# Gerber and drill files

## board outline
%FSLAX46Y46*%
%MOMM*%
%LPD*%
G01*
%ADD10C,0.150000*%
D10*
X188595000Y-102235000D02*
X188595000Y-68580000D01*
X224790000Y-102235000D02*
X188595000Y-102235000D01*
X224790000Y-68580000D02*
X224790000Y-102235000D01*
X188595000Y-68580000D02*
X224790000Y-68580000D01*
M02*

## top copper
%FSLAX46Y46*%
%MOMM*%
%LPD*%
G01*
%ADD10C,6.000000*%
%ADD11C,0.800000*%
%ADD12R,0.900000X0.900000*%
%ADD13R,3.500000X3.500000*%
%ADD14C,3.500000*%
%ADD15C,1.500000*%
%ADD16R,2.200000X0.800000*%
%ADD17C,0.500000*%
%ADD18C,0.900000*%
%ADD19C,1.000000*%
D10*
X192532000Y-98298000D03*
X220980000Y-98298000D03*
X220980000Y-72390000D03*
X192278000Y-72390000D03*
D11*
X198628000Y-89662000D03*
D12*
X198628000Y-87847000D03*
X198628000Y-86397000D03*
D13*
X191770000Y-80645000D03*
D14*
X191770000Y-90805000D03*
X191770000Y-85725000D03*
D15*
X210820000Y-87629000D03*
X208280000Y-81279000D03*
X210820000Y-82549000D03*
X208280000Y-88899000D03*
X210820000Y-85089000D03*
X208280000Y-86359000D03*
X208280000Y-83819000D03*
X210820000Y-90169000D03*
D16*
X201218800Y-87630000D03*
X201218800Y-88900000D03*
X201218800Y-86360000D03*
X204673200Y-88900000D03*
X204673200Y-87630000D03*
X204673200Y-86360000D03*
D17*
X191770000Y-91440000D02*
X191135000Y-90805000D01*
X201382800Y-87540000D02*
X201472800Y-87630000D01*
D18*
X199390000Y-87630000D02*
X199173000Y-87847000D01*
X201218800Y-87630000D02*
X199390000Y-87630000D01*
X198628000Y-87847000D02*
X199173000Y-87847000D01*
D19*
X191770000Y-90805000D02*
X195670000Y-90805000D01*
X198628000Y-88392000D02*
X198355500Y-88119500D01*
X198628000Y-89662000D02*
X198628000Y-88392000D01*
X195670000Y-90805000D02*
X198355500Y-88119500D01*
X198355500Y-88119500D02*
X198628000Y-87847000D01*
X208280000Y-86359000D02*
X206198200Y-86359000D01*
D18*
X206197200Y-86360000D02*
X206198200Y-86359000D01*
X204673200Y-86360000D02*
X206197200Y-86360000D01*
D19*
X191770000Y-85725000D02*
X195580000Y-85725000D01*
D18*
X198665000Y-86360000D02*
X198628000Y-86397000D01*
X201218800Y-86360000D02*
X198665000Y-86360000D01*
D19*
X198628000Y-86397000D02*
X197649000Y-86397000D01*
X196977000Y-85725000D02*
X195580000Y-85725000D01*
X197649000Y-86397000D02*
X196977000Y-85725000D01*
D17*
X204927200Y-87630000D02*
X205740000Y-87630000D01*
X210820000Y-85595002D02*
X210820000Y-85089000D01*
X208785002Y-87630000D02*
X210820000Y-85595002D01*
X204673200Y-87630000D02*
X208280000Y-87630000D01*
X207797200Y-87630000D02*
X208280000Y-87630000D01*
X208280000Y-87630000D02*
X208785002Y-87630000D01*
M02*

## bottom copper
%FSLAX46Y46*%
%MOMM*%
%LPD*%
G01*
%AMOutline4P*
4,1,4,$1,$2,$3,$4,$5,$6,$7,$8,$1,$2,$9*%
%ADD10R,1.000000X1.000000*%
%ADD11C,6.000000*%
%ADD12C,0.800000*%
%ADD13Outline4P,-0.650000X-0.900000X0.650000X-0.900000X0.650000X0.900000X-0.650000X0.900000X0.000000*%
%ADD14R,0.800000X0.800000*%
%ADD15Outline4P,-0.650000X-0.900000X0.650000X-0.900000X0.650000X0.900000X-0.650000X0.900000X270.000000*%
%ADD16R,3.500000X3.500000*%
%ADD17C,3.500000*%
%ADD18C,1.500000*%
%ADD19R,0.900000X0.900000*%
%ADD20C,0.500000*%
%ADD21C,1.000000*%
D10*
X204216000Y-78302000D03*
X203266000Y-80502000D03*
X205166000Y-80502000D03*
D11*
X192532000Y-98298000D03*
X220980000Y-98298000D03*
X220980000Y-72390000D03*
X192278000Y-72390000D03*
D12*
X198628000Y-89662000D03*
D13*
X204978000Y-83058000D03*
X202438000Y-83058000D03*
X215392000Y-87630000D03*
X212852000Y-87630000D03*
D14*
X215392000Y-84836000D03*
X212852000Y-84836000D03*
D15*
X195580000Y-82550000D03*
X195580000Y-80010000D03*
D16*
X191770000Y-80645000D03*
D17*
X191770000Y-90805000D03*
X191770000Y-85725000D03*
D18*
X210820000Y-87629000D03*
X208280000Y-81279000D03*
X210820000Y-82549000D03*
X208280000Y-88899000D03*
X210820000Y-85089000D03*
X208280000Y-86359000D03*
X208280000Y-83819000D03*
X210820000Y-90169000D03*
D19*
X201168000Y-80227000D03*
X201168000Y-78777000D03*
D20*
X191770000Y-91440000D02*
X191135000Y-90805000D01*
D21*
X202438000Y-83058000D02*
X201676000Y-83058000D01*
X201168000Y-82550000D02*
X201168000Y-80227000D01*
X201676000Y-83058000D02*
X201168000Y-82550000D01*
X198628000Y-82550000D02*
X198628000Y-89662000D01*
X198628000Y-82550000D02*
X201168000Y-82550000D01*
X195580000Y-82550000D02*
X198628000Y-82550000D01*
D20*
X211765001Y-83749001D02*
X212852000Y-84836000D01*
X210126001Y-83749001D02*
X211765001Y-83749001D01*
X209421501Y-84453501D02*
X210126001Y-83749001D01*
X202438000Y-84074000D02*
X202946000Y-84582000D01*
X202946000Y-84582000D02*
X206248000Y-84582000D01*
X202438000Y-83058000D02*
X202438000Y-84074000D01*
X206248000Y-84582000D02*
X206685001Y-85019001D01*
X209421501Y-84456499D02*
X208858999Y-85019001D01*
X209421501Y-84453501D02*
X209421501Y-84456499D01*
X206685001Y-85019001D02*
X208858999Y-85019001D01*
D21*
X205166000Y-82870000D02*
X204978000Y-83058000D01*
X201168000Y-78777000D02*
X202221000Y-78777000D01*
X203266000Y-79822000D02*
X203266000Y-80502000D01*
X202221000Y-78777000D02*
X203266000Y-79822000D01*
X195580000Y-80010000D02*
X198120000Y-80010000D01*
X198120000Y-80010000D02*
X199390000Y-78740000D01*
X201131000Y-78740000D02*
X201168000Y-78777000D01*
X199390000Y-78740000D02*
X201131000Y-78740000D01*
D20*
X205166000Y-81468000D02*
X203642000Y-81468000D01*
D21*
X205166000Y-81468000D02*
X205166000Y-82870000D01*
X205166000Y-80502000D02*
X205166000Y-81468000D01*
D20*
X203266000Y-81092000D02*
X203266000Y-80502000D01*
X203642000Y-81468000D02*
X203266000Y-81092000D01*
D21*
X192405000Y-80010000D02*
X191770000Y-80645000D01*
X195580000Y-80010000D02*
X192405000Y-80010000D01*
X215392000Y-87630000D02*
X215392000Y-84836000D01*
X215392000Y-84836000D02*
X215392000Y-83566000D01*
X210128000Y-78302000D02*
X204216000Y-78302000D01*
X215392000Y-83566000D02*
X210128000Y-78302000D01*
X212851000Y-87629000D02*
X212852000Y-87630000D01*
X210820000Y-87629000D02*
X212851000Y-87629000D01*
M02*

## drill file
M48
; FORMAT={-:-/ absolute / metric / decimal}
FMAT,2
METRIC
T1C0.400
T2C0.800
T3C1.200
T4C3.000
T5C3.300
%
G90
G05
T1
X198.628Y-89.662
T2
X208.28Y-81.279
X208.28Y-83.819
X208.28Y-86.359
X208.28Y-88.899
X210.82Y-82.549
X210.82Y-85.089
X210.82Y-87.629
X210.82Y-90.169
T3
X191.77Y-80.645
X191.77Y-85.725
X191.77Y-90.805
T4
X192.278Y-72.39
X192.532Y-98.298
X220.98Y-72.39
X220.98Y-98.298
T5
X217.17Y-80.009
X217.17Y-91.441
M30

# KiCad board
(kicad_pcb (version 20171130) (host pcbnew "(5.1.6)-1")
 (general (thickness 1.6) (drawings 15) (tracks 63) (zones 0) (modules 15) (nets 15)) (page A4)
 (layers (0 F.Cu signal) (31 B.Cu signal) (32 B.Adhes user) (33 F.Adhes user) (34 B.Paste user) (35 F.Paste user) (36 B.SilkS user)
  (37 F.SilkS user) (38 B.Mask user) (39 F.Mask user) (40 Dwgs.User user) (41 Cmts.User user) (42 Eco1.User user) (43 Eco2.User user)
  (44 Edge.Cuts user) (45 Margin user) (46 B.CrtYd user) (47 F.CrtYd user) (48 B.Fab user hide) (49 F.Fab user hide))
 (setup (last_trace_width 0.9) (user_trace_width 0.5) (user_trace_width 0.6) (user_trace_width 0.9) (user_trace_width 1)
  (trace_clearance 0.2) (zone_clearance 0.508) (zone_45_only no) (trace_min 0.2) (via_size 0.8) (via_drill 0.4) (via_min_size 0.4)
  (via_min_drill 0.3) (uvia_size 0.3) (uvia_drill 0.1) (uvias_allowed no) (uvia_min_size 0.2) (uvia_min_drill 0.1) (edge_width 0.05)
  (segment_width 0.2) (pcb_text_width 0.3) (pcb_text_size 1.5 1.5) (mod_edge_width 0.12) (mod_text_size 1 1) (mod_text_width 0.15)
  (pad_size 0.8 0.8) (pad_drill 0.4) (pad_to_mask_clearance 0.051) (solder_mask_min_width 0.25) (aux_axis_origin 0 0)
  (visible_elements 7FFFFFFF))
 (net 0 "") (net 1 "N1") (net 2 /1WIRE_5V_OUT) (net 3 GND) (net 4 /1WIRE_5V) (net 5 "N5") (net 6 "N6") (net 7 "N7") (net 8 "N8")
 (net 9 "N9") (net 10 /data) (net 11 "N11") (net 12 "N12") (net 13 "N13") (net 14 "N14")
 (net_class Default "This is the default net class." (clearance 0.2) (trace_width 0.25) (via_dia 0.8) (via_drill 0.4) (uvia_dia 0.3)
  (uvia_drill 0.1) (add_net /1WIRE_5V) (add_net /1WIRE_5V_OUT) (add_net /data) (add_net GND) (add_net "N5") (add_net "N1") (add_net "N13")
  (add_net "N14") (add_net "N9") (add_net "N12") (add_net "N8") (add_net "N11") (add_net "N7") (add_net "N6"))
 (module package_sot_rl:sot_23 (layer B.Cu) (at 204.216 79.502 90)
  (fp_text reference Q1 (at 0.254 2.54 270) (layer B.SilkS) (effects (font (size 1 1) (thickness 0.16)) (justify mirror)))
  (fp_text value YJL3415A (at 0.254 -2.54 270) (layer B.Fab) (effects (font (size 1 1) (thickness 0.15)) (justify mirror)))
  (pad 3 smd rect (at 1.2 0 90) (size 1 1) (layers B.Cu B.Paste B.Mask) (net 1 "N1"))
  (pad 2 smd rect (at -1 -0.95 90) (size 1 1) (layers B.Cu B.Paste B.Mask) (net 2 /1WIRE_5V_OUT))
  (pad 1 smd rect (at -1 0.95 90) (size 1 1) (layers B.Cu B.Paste B.Mask) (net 2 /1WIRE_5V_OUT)))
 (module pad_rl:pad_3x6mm (layer F.Cu) (at 192.532 98.298)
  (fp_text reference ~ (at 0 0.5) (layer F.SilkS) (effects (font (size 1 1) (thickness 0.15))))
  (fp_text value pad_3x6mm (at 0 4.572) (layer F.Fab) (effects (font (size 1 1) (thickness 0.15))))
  (pad ~ thru_hole circle (at 0 0) (size 6 6) (drill 3) (layers *.Cu *.Mask)))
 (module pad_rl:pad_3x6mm (layer F.Cu) (at 220.98 98.298)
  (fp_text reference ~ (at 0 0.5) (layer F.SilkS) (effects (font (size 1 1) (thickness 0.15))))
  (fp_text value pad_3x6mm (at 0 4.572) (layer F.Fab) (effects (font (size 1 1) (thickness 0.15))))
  (pad ~ thru_hole circle (at 0 0) (size 6 6) (drill 3) (layers *.Cu *.Mask)))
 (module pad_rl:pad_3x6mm (layer F.Cu) (at 220.98 72.39)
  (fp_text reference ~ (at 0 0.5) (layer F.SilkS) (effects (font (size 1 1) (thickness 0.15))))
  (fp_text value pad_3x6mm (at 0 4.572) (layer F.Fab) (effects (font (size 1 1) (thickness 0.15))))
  (pad ~ thru_hole circle (at 0 0) (size 6 6) (drill 3) (layers *.Cu *.Mask)))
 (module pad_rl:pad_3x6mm (layer F.Cu) (at 192.278 72.39)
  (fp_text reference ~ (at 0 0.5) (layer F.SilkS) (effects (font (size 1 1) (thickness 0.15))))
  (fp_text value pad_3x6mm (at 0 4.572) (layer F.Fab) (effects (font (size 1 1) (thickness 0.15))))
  (pad ~ thru_hole circle (at 0 0) (size 6 6) (drill 3) (layers *.Cu *.Mask)))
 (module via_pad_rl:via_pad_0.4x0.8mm (layer F.Cu) (at 198.628 89.662)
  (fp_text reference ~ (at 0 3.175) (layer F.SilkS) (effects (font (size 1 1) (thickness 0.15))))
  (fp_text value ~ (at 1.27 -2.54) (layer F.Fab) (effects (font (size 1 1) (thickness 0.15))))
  (pad ~ thru_hole circle (at 0 0) (size 0.8 0.8) (drill 0.4) (layers *.Cu *.Mask) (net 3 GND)))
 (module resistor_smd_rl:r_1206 (layer B.Cu) (at 203.708 83.058)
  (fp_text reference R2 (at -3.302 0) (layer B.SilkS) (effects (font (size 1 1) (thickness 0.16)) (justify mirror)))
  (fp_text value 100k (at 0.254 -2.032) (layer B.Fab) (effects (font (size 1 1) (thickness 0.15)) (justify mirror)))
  (pad 2 smd trapezoid (at 1.27 0) (size 1.3 1.8) (layers B.Cu B.Paste B.Mask) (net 2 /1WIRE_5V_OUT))
  (pad 1 smd trapezoid (at -1.27 0) (size 1.3 1.8) (layers B.Cu B.Paste B.Mask) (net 3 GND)))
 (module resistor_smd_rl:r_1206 (layer B.Cu) (at 214.122 87.63)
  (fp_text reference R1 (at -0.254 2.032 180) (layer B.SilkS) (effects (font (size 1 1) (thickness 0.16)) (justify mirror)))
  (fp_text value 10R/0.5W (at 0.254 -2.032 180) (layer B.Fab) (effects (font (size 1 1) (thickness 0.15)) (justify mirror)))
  (pad 2 smd trapezoid (at 1.27 0) (size 1.3 1.8) (layers B.Cu B.Paste B.Mask) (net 1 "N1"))
  (pad 1 smd trapezoid (at -1.27 0) (size 1.3 1.8) (layers B.Cu B.Paste B.Mask) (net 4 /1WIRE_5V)))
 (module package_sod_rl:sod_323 (layer B.Cu) (at 214.122 84.836 180)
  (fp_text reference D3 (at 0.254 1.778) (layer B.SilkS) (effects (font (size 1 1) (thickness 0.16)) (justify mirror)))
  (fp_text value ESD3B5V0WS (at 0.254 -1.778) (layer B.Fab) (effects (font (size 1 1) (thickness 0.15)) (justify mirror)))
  (pad 1 smd rect (at -1.27 0 180) (size 0.8 0.8) (layers B.Cu B.Paste B.Mask) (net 1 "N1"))
  (pad 2 smd rect (at 1.27 0 180) (size 0.8 0.8) (layers B.Cu B.Paste B.Mask) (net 3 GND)))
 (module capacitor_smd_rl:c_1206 (layer B.Cu) (at 195.58 81.28 270)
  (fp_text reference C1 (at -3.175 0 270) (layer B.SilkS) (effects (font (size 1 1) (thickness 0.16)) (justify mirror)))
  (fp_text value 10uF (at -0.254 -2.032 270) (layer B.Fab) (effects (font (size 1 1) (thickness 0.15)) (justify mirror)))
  (pad 2 smd trapezoid (at 1.27 0 270) (size 1.3 1.8) (layers B.Cu B.Paste B.Mask) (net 3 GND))
  (pad 1 smd trapezoid (at -1.27 0 270) (size 1.3 1.8) (layers B.Cu B.Paste B.Mask) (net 2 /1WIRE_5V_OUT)))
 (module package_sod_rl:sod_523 (layer F.Cu) (at 198.628 87.122 270)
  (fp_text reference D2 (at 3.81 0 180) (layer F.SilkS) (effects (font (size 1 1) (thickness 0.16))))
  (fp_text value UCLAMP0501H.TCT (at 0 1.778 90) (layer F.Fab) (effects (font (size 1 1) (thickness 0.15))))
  (pad 2 smd rect (at 0.725 0 270) (size 0.9 0.9) (layers F.Cu F.Paste F.Mask) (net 3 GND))
  (pad 1 smd rect (at -0.725 0 270) (size 0.9 0.9) (layers F.Cu F.Paste F.Mask) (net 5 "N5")))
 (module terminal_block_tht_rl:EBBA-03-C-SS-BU (layer F.Cu) (at 191.77 85.725 270)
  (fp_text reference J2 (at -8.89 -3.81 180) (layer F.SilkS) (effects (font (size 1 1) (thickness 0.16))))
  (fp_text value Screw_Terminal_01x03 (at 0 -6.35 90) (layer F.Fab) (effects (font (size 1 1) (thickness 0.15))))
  (pad 1 thru_hole rect (at -5.08 0 90) (size 3.5 3.5) (drill 1.2) (layers *.Cu *.Mask) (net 2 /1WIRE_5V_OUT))
  (pad 3 thru_hole circle (at 5.08 0 90) (size 3.5 3.5) (drill 1.2) (layers *.Cu *.Mask) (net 3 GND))
  (pad 2 thru_hole circle (at 0 0 90) (size 3.5 3.5) (drill 1.2) (layers *.Cu *.Mask) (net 5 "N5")))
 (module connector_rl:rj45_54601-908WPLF (layer F.Cu) (at 217.17 85.725 90)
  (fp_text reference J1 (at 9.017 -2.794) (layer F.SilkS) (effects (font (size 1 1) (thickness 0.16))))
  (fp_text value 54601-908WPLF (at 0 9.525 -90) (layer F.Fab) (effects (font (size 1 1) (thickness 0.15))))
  (pad 3 thru_hole circle (at -1.904 -6.35 90) (size 1.5 1.5) (drill 0.8) (layers *.Cu *.Mask) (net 4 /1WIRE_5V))
  (pad 8 thru_hole circle (at 4.446 -8.89 90) (size 1.5 1.5) (drill 0.8) (layers *.Cu *.Mask) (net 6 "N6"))
  (pad "" np_thru_hole circle (at -5.716 0 90) (size 3.3 3.3) (drill 3.3) (layers *.Cu *.SilkS *.Mask))
  (pad 7 thru_hole circle (at 3.176 -6.35 90) (size 1.5 1.5) (drill 0.8) (layers *.Cu *.Mask) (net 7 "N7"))
  (pad 2 thru_hole circle (at -3.174 -8.89 90) (size 1.5 1.5) (drill 0.8) (layers *.Cu *.Mask) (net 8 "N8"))
  (pad 5 thru_hole circle (at 0.636 -6.35 90) (size 1.5 1.5) (drill 0.8) (layers *.Cu *.Mask) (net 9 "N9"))
  (pad 4 thru_hole circle (at -0.634 -8.89 90) (size 1.5 1.5) (drill 0.8) (layers *.Cu *.Mask) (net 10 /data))
  (pad 6 thru_hole circle (at 1.906 -8.89 270) (size 1.5 1.5) (drill 0.8) (layers *.Cu *.Mask) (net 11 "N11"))
  (pad 1 thru_hole circle (at -4.444 -6.35 90) (size 1.5 1.5) (drill 0.8) (layers *.Cu *.Mask) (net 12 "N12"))
  (pad "" np_thru_hole circle (at 5.716 0 90) (size 3.3 3.3) (drill 3.3) (layers *.Cu *.SilkS *.Mask)))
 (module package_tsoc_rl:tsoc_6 (layer F.Cu) (at 202.946 87.63)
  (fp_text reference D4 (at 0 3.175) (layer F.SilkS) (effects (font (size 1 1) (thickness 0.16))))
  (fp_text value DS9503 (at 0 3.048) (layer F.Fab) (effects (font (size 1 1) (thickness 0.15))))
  (pad 2 smd rect (at -1.7272 0) (size 2.2 0.8) (layers F.Cu F.Paste F.Mask) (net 3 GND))
  (pad 3 smd rect (at -1.7272 1.27) (size 2.2 0.8) (layers F.Cu F.Paste F.Mask) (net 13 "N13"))
  (pad 1 smd rect (at -1.7272 -1.27) (size 2.2 0.8) (layers F.Cu F.Paste F.Mask) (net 5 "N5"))
  (pad 4 smd rect (at 1.7272 1.27) (size 2.2 0.8) (layers F.Cu F.Paste F.Mask) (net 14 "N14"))
  (pad 5 smd rect (at 1.7272 0) (size 2.2 0.8) (layers F.Cu F.Paste F.Mask) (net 9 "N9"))
  (pad 6 smd rect (at 1.7272 -1.27) (size 2.2 0.8) (layers F.Cu F.Paste F.Mask) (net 10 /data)))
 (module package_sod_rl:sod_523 (layer B.Cu) (at 201.168 79.502 270)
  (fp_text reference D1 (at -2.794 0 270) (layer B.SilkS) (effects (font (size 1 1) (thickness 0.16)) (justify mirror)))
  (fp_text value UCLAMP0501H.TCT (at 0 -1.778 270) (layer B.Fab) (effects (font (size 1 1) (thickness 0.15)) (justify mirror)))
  (pad 2 smd rect (at 0.725 0 270) (size 0.9 0.9) (layers B.Cu B.Paste B.Mask) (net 3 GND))
  (pad 1 smd rect (at -0.725 0 270) (size 0.9 0.9) (layers B.Cu B.Paste B.Mask) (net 2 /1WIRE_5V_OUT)))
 (gr_line (start 188.595 102.235) (end 188.595 68.58) (layer Edge.Cuts) (width 0.15))
 (gr_line (start 224.79 102.235) (end 188.595 102.235) (layer Edge.Cuts) (width 0.15))
 (gr_line (start 224.79 68.58) (end 224.79 102.235) (layer Edge.Cuts) (width 0.15))
 (gr_line (start 188.595 68.58) (end 224.79 68.58) (layer Edge.Cuts) (width 0.15))
 (segment (start 191.77 91.44) (end 191.135 90.805) (width 0.5) (layer F.Cu) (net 3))
 (segment (start 191.77 91.44) (end 191.135 90.805) (width 0.5) (layer B.Cu) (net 3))
 (segment (start 201.3828 87.54) (end 201.4728 87.63) (width 0.5) (layer F.Cu) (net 3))
 (segment (start 202.438 83.058) (end 201.676 83.058) (width 1) (layer B.Cu) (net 3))
 (segment (start 201.168 82.55) (end 201.168 80.227) (width 1) (layer B.Cu) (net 3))
 (segment (start 201.676 83.058) (end 201.168 82.55) (width 1) (layer B.Cu) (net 3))
 (segment (start 199.39 87.63) (end 199.173 87.847) (width 0.9) (layer F.Cu) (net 3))
 (segment (start 201.2188 87.63) (end 199.39 87.63) (width 0.9) (layer F.Cu) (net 3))
 (segment (start 198.628 87.847) (end 199.173 87.847) (width 0.9) (layer F.Cu) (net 3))
 (segment (start 191.77 90.805) (end 195.67 90.805) (width 1) (layer F.Cu) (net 3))
 (segment (start 198.628 82.55) (end 198.628 89.662) (width 1) (layer B.Cu) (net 3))
 (segment (start 198.628 82.55) (end 201.168 82.55) (width 1) (layer B.Cu) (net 3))
 (segment (start 195.58 82.55) (end 198.628 82.55) (width 1) (layer B.Cu) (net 3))
 (segment (start 198.628 88.392) (end 198.3555 88.1195) (width 1) (layer F.Cu) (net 3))
 (segment (start 198.628 89.662) (end 198.628 88.392) (width 1) (layer F.Cu) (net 3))
 (segment (start 195.67 90.805) (end 198.3555 88.1195) (width 1) (layer F.Cu) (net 3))
 (segment (start 198.3555 88.1195) (end 198.628 87.847) (width 1) (layer F.Cu) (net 3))
 (segment (start 211.765001 83.749001) (end 212.852 84.836) (width 0.5) (layer B.Cu) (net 3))
 (segment (start 210.126001 83.749001) (end 211.765001 83.749001) (width 0.5) (layer B.Cu) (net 3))
 (segment (start 209.421501 84.453501) (end 210.126001 83.749001) (width 0.5) (layer B.Cu) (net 3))
 (segment (start 202.438 84.074) (end 202.946 84.582) (width 0.5) (layer B.Cu) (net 3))
 (segment (start 202.946 84.582) (end 206.248 84.582) (width 0.5) (layer B.Cu) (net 3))
 (segment (start 202.438 83.058) (end 202.438 84.074) (width 0.5) (layer B.Cu) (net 3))
 (segment (start 206.248 84.582) (end 206.685001 85.019001) (width 0.5) (layer B.Cu) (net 3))
 (segment (start 209.421501 84.456499) (end 208.858999 85.019001) (width 0.5) (layer B.Cu) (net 3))
 (segment (start 209.421501 84.453501) (end 209.421501 84.456499) (width 0.5) (layer B.Cu) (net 3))
 (segment (start 206.685001 85.019001) (end 208.858999 85.019001) (width 0.5) (layer B.Cu) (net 3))
 (segment (start 208.28 86.359) (end 206.1982 86.359) (width 1) (layer F.Cu) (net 10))
 (segment (start 206.1972 86.36) (end 206.1982 86.359) (width 0.9) (layer F.Cu) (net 10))
 (segment (start 204.6732 86.36) (end 206.1972 86.36) (width 0.9) (layer F.Cu) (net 10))
 (segment (start 191.77 85.725) (end 195.58 85.725) (width 1) (layer F.Cu) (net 5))
 (segment (start 198.665 86.36) (end 198.628 86.397) (width 0.9) (layer F.Cu) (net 5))
 (segment (start 201.2188 86.36) (end 198.665 86.36) (width 0.9) (layer F.Cu) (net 5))
 (segment (start 198.628 86.397) (end 197.649 86.397) (width 1) (layer F.Cu) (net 5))
 (segment (start 196.977 85.725) (end 195.58 85.725) (width 1) (layer F.Cu) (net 5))
 (segment (start 197.649 86.397) (end 196.977 85.725) (width 1) (layer F.Cu) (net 5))
 (segment (start 205.166 82.87) (end 204.978 83.058) (width 1) (layer B.Cu) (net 2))
 (segment (start 201.168 78.777) (end 202.221 78.777) (width 1) (layer B.Cu) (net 2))
 (segment (start 203.266 79.822) (end 203.266 80.502) (width 1) (layer B.Cu) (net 2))
 (segment (start 202.221 78.777) (end 203.266 79.822) (width 1) (layer B.Cu) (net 2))
 (segment (start 195.58 80.01) (end 198.12 80.01) (width 1) (layer B.Cu) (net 2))
 (segment (start 198.12 80.01) (end 199.39 78.74) (width 1) (layer B.Cu) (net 2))
 (segment (start 201.131 78.74) (end 201.168 78.777) (width 1) (layer B.Cu) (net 2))
 (segment (start 199.39 78.74) (end 201.131 78.74) (width 1) (layer B.Cu) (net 2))
 (segment (start 205.166 81.468) (end 203.642 81.468) (width 0.5) (layer B.Cu) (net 2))
 (segment (start 205.166 81.468) (end 205.166 82.87) (width 1) (layer B.Cu) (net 2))
 (segment (start 205.166 80.502) (end 205.166 81.468) (width 1) (layer B.Cu) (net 2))
 (segment (start 203.266 81.092) (end 203.266 80.502) (width 0.5) (layer B.Cu) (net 2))
 (segment (start 203.642 81.468) (end 203.266 81.092) (width 0.5) (layer B.Cu) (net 2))
 (segment (start 192.405 80.01) (end 191.77 80.645) (width 1) (layer B.Cu) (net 2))
 (segment (start 195.58 80.01) (end 192.405 80.01) (width 1) (layer B.Cu) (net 2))
 (segment (start 215.392 87.63) (end 215.392 84.836) (width 1) (layer B.Cu) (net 1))
 (segment (start 215.392 84.836) (end 215.392 83.566) (width 1) (layer B.Cu) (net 1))
 (segment (start 210.128 78.302) (end 204.216 78.302) (width 1) (layer B.Cu) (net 1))
 (segment (start 215.392 83.566) (end 210.128 78.302) (width 1) (layer B.Cu) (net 1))
 (segment (start 204.9272 87.63) (end 205.74 87.63) (width 0.5) (layer F.Cu) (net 9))
 (segment (start 210.82 85.595002) (end 210.82 85.089) (width 0.5) (layer F.Cu) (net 9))
 (segment (start 208.785002 87.63) (end 210.82 85.595002) (width 0.5) (layer F.Cu) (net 9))
 (segment (start 204.6732 87.63) (end 208.28 87.63) (width 0.5) (layer F.Cu) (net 9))
 (segment (start 207.7972 87.63) (end 208.28 87.63) (width 0.5) (layer F.Cu) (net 9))
 (segment (start 208.28 87.63) (end 208.785002 87.63) (width 0.5) (layer F.Cu) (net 9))
 (segment (start 212.851 87.629) (end 212.852 87.63) (width 1) (layer B.Cu) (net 4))
 (segment (start 210.82 87.629) (end 212.851 87.629) (width 1) (layer B.Cu) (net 4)))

